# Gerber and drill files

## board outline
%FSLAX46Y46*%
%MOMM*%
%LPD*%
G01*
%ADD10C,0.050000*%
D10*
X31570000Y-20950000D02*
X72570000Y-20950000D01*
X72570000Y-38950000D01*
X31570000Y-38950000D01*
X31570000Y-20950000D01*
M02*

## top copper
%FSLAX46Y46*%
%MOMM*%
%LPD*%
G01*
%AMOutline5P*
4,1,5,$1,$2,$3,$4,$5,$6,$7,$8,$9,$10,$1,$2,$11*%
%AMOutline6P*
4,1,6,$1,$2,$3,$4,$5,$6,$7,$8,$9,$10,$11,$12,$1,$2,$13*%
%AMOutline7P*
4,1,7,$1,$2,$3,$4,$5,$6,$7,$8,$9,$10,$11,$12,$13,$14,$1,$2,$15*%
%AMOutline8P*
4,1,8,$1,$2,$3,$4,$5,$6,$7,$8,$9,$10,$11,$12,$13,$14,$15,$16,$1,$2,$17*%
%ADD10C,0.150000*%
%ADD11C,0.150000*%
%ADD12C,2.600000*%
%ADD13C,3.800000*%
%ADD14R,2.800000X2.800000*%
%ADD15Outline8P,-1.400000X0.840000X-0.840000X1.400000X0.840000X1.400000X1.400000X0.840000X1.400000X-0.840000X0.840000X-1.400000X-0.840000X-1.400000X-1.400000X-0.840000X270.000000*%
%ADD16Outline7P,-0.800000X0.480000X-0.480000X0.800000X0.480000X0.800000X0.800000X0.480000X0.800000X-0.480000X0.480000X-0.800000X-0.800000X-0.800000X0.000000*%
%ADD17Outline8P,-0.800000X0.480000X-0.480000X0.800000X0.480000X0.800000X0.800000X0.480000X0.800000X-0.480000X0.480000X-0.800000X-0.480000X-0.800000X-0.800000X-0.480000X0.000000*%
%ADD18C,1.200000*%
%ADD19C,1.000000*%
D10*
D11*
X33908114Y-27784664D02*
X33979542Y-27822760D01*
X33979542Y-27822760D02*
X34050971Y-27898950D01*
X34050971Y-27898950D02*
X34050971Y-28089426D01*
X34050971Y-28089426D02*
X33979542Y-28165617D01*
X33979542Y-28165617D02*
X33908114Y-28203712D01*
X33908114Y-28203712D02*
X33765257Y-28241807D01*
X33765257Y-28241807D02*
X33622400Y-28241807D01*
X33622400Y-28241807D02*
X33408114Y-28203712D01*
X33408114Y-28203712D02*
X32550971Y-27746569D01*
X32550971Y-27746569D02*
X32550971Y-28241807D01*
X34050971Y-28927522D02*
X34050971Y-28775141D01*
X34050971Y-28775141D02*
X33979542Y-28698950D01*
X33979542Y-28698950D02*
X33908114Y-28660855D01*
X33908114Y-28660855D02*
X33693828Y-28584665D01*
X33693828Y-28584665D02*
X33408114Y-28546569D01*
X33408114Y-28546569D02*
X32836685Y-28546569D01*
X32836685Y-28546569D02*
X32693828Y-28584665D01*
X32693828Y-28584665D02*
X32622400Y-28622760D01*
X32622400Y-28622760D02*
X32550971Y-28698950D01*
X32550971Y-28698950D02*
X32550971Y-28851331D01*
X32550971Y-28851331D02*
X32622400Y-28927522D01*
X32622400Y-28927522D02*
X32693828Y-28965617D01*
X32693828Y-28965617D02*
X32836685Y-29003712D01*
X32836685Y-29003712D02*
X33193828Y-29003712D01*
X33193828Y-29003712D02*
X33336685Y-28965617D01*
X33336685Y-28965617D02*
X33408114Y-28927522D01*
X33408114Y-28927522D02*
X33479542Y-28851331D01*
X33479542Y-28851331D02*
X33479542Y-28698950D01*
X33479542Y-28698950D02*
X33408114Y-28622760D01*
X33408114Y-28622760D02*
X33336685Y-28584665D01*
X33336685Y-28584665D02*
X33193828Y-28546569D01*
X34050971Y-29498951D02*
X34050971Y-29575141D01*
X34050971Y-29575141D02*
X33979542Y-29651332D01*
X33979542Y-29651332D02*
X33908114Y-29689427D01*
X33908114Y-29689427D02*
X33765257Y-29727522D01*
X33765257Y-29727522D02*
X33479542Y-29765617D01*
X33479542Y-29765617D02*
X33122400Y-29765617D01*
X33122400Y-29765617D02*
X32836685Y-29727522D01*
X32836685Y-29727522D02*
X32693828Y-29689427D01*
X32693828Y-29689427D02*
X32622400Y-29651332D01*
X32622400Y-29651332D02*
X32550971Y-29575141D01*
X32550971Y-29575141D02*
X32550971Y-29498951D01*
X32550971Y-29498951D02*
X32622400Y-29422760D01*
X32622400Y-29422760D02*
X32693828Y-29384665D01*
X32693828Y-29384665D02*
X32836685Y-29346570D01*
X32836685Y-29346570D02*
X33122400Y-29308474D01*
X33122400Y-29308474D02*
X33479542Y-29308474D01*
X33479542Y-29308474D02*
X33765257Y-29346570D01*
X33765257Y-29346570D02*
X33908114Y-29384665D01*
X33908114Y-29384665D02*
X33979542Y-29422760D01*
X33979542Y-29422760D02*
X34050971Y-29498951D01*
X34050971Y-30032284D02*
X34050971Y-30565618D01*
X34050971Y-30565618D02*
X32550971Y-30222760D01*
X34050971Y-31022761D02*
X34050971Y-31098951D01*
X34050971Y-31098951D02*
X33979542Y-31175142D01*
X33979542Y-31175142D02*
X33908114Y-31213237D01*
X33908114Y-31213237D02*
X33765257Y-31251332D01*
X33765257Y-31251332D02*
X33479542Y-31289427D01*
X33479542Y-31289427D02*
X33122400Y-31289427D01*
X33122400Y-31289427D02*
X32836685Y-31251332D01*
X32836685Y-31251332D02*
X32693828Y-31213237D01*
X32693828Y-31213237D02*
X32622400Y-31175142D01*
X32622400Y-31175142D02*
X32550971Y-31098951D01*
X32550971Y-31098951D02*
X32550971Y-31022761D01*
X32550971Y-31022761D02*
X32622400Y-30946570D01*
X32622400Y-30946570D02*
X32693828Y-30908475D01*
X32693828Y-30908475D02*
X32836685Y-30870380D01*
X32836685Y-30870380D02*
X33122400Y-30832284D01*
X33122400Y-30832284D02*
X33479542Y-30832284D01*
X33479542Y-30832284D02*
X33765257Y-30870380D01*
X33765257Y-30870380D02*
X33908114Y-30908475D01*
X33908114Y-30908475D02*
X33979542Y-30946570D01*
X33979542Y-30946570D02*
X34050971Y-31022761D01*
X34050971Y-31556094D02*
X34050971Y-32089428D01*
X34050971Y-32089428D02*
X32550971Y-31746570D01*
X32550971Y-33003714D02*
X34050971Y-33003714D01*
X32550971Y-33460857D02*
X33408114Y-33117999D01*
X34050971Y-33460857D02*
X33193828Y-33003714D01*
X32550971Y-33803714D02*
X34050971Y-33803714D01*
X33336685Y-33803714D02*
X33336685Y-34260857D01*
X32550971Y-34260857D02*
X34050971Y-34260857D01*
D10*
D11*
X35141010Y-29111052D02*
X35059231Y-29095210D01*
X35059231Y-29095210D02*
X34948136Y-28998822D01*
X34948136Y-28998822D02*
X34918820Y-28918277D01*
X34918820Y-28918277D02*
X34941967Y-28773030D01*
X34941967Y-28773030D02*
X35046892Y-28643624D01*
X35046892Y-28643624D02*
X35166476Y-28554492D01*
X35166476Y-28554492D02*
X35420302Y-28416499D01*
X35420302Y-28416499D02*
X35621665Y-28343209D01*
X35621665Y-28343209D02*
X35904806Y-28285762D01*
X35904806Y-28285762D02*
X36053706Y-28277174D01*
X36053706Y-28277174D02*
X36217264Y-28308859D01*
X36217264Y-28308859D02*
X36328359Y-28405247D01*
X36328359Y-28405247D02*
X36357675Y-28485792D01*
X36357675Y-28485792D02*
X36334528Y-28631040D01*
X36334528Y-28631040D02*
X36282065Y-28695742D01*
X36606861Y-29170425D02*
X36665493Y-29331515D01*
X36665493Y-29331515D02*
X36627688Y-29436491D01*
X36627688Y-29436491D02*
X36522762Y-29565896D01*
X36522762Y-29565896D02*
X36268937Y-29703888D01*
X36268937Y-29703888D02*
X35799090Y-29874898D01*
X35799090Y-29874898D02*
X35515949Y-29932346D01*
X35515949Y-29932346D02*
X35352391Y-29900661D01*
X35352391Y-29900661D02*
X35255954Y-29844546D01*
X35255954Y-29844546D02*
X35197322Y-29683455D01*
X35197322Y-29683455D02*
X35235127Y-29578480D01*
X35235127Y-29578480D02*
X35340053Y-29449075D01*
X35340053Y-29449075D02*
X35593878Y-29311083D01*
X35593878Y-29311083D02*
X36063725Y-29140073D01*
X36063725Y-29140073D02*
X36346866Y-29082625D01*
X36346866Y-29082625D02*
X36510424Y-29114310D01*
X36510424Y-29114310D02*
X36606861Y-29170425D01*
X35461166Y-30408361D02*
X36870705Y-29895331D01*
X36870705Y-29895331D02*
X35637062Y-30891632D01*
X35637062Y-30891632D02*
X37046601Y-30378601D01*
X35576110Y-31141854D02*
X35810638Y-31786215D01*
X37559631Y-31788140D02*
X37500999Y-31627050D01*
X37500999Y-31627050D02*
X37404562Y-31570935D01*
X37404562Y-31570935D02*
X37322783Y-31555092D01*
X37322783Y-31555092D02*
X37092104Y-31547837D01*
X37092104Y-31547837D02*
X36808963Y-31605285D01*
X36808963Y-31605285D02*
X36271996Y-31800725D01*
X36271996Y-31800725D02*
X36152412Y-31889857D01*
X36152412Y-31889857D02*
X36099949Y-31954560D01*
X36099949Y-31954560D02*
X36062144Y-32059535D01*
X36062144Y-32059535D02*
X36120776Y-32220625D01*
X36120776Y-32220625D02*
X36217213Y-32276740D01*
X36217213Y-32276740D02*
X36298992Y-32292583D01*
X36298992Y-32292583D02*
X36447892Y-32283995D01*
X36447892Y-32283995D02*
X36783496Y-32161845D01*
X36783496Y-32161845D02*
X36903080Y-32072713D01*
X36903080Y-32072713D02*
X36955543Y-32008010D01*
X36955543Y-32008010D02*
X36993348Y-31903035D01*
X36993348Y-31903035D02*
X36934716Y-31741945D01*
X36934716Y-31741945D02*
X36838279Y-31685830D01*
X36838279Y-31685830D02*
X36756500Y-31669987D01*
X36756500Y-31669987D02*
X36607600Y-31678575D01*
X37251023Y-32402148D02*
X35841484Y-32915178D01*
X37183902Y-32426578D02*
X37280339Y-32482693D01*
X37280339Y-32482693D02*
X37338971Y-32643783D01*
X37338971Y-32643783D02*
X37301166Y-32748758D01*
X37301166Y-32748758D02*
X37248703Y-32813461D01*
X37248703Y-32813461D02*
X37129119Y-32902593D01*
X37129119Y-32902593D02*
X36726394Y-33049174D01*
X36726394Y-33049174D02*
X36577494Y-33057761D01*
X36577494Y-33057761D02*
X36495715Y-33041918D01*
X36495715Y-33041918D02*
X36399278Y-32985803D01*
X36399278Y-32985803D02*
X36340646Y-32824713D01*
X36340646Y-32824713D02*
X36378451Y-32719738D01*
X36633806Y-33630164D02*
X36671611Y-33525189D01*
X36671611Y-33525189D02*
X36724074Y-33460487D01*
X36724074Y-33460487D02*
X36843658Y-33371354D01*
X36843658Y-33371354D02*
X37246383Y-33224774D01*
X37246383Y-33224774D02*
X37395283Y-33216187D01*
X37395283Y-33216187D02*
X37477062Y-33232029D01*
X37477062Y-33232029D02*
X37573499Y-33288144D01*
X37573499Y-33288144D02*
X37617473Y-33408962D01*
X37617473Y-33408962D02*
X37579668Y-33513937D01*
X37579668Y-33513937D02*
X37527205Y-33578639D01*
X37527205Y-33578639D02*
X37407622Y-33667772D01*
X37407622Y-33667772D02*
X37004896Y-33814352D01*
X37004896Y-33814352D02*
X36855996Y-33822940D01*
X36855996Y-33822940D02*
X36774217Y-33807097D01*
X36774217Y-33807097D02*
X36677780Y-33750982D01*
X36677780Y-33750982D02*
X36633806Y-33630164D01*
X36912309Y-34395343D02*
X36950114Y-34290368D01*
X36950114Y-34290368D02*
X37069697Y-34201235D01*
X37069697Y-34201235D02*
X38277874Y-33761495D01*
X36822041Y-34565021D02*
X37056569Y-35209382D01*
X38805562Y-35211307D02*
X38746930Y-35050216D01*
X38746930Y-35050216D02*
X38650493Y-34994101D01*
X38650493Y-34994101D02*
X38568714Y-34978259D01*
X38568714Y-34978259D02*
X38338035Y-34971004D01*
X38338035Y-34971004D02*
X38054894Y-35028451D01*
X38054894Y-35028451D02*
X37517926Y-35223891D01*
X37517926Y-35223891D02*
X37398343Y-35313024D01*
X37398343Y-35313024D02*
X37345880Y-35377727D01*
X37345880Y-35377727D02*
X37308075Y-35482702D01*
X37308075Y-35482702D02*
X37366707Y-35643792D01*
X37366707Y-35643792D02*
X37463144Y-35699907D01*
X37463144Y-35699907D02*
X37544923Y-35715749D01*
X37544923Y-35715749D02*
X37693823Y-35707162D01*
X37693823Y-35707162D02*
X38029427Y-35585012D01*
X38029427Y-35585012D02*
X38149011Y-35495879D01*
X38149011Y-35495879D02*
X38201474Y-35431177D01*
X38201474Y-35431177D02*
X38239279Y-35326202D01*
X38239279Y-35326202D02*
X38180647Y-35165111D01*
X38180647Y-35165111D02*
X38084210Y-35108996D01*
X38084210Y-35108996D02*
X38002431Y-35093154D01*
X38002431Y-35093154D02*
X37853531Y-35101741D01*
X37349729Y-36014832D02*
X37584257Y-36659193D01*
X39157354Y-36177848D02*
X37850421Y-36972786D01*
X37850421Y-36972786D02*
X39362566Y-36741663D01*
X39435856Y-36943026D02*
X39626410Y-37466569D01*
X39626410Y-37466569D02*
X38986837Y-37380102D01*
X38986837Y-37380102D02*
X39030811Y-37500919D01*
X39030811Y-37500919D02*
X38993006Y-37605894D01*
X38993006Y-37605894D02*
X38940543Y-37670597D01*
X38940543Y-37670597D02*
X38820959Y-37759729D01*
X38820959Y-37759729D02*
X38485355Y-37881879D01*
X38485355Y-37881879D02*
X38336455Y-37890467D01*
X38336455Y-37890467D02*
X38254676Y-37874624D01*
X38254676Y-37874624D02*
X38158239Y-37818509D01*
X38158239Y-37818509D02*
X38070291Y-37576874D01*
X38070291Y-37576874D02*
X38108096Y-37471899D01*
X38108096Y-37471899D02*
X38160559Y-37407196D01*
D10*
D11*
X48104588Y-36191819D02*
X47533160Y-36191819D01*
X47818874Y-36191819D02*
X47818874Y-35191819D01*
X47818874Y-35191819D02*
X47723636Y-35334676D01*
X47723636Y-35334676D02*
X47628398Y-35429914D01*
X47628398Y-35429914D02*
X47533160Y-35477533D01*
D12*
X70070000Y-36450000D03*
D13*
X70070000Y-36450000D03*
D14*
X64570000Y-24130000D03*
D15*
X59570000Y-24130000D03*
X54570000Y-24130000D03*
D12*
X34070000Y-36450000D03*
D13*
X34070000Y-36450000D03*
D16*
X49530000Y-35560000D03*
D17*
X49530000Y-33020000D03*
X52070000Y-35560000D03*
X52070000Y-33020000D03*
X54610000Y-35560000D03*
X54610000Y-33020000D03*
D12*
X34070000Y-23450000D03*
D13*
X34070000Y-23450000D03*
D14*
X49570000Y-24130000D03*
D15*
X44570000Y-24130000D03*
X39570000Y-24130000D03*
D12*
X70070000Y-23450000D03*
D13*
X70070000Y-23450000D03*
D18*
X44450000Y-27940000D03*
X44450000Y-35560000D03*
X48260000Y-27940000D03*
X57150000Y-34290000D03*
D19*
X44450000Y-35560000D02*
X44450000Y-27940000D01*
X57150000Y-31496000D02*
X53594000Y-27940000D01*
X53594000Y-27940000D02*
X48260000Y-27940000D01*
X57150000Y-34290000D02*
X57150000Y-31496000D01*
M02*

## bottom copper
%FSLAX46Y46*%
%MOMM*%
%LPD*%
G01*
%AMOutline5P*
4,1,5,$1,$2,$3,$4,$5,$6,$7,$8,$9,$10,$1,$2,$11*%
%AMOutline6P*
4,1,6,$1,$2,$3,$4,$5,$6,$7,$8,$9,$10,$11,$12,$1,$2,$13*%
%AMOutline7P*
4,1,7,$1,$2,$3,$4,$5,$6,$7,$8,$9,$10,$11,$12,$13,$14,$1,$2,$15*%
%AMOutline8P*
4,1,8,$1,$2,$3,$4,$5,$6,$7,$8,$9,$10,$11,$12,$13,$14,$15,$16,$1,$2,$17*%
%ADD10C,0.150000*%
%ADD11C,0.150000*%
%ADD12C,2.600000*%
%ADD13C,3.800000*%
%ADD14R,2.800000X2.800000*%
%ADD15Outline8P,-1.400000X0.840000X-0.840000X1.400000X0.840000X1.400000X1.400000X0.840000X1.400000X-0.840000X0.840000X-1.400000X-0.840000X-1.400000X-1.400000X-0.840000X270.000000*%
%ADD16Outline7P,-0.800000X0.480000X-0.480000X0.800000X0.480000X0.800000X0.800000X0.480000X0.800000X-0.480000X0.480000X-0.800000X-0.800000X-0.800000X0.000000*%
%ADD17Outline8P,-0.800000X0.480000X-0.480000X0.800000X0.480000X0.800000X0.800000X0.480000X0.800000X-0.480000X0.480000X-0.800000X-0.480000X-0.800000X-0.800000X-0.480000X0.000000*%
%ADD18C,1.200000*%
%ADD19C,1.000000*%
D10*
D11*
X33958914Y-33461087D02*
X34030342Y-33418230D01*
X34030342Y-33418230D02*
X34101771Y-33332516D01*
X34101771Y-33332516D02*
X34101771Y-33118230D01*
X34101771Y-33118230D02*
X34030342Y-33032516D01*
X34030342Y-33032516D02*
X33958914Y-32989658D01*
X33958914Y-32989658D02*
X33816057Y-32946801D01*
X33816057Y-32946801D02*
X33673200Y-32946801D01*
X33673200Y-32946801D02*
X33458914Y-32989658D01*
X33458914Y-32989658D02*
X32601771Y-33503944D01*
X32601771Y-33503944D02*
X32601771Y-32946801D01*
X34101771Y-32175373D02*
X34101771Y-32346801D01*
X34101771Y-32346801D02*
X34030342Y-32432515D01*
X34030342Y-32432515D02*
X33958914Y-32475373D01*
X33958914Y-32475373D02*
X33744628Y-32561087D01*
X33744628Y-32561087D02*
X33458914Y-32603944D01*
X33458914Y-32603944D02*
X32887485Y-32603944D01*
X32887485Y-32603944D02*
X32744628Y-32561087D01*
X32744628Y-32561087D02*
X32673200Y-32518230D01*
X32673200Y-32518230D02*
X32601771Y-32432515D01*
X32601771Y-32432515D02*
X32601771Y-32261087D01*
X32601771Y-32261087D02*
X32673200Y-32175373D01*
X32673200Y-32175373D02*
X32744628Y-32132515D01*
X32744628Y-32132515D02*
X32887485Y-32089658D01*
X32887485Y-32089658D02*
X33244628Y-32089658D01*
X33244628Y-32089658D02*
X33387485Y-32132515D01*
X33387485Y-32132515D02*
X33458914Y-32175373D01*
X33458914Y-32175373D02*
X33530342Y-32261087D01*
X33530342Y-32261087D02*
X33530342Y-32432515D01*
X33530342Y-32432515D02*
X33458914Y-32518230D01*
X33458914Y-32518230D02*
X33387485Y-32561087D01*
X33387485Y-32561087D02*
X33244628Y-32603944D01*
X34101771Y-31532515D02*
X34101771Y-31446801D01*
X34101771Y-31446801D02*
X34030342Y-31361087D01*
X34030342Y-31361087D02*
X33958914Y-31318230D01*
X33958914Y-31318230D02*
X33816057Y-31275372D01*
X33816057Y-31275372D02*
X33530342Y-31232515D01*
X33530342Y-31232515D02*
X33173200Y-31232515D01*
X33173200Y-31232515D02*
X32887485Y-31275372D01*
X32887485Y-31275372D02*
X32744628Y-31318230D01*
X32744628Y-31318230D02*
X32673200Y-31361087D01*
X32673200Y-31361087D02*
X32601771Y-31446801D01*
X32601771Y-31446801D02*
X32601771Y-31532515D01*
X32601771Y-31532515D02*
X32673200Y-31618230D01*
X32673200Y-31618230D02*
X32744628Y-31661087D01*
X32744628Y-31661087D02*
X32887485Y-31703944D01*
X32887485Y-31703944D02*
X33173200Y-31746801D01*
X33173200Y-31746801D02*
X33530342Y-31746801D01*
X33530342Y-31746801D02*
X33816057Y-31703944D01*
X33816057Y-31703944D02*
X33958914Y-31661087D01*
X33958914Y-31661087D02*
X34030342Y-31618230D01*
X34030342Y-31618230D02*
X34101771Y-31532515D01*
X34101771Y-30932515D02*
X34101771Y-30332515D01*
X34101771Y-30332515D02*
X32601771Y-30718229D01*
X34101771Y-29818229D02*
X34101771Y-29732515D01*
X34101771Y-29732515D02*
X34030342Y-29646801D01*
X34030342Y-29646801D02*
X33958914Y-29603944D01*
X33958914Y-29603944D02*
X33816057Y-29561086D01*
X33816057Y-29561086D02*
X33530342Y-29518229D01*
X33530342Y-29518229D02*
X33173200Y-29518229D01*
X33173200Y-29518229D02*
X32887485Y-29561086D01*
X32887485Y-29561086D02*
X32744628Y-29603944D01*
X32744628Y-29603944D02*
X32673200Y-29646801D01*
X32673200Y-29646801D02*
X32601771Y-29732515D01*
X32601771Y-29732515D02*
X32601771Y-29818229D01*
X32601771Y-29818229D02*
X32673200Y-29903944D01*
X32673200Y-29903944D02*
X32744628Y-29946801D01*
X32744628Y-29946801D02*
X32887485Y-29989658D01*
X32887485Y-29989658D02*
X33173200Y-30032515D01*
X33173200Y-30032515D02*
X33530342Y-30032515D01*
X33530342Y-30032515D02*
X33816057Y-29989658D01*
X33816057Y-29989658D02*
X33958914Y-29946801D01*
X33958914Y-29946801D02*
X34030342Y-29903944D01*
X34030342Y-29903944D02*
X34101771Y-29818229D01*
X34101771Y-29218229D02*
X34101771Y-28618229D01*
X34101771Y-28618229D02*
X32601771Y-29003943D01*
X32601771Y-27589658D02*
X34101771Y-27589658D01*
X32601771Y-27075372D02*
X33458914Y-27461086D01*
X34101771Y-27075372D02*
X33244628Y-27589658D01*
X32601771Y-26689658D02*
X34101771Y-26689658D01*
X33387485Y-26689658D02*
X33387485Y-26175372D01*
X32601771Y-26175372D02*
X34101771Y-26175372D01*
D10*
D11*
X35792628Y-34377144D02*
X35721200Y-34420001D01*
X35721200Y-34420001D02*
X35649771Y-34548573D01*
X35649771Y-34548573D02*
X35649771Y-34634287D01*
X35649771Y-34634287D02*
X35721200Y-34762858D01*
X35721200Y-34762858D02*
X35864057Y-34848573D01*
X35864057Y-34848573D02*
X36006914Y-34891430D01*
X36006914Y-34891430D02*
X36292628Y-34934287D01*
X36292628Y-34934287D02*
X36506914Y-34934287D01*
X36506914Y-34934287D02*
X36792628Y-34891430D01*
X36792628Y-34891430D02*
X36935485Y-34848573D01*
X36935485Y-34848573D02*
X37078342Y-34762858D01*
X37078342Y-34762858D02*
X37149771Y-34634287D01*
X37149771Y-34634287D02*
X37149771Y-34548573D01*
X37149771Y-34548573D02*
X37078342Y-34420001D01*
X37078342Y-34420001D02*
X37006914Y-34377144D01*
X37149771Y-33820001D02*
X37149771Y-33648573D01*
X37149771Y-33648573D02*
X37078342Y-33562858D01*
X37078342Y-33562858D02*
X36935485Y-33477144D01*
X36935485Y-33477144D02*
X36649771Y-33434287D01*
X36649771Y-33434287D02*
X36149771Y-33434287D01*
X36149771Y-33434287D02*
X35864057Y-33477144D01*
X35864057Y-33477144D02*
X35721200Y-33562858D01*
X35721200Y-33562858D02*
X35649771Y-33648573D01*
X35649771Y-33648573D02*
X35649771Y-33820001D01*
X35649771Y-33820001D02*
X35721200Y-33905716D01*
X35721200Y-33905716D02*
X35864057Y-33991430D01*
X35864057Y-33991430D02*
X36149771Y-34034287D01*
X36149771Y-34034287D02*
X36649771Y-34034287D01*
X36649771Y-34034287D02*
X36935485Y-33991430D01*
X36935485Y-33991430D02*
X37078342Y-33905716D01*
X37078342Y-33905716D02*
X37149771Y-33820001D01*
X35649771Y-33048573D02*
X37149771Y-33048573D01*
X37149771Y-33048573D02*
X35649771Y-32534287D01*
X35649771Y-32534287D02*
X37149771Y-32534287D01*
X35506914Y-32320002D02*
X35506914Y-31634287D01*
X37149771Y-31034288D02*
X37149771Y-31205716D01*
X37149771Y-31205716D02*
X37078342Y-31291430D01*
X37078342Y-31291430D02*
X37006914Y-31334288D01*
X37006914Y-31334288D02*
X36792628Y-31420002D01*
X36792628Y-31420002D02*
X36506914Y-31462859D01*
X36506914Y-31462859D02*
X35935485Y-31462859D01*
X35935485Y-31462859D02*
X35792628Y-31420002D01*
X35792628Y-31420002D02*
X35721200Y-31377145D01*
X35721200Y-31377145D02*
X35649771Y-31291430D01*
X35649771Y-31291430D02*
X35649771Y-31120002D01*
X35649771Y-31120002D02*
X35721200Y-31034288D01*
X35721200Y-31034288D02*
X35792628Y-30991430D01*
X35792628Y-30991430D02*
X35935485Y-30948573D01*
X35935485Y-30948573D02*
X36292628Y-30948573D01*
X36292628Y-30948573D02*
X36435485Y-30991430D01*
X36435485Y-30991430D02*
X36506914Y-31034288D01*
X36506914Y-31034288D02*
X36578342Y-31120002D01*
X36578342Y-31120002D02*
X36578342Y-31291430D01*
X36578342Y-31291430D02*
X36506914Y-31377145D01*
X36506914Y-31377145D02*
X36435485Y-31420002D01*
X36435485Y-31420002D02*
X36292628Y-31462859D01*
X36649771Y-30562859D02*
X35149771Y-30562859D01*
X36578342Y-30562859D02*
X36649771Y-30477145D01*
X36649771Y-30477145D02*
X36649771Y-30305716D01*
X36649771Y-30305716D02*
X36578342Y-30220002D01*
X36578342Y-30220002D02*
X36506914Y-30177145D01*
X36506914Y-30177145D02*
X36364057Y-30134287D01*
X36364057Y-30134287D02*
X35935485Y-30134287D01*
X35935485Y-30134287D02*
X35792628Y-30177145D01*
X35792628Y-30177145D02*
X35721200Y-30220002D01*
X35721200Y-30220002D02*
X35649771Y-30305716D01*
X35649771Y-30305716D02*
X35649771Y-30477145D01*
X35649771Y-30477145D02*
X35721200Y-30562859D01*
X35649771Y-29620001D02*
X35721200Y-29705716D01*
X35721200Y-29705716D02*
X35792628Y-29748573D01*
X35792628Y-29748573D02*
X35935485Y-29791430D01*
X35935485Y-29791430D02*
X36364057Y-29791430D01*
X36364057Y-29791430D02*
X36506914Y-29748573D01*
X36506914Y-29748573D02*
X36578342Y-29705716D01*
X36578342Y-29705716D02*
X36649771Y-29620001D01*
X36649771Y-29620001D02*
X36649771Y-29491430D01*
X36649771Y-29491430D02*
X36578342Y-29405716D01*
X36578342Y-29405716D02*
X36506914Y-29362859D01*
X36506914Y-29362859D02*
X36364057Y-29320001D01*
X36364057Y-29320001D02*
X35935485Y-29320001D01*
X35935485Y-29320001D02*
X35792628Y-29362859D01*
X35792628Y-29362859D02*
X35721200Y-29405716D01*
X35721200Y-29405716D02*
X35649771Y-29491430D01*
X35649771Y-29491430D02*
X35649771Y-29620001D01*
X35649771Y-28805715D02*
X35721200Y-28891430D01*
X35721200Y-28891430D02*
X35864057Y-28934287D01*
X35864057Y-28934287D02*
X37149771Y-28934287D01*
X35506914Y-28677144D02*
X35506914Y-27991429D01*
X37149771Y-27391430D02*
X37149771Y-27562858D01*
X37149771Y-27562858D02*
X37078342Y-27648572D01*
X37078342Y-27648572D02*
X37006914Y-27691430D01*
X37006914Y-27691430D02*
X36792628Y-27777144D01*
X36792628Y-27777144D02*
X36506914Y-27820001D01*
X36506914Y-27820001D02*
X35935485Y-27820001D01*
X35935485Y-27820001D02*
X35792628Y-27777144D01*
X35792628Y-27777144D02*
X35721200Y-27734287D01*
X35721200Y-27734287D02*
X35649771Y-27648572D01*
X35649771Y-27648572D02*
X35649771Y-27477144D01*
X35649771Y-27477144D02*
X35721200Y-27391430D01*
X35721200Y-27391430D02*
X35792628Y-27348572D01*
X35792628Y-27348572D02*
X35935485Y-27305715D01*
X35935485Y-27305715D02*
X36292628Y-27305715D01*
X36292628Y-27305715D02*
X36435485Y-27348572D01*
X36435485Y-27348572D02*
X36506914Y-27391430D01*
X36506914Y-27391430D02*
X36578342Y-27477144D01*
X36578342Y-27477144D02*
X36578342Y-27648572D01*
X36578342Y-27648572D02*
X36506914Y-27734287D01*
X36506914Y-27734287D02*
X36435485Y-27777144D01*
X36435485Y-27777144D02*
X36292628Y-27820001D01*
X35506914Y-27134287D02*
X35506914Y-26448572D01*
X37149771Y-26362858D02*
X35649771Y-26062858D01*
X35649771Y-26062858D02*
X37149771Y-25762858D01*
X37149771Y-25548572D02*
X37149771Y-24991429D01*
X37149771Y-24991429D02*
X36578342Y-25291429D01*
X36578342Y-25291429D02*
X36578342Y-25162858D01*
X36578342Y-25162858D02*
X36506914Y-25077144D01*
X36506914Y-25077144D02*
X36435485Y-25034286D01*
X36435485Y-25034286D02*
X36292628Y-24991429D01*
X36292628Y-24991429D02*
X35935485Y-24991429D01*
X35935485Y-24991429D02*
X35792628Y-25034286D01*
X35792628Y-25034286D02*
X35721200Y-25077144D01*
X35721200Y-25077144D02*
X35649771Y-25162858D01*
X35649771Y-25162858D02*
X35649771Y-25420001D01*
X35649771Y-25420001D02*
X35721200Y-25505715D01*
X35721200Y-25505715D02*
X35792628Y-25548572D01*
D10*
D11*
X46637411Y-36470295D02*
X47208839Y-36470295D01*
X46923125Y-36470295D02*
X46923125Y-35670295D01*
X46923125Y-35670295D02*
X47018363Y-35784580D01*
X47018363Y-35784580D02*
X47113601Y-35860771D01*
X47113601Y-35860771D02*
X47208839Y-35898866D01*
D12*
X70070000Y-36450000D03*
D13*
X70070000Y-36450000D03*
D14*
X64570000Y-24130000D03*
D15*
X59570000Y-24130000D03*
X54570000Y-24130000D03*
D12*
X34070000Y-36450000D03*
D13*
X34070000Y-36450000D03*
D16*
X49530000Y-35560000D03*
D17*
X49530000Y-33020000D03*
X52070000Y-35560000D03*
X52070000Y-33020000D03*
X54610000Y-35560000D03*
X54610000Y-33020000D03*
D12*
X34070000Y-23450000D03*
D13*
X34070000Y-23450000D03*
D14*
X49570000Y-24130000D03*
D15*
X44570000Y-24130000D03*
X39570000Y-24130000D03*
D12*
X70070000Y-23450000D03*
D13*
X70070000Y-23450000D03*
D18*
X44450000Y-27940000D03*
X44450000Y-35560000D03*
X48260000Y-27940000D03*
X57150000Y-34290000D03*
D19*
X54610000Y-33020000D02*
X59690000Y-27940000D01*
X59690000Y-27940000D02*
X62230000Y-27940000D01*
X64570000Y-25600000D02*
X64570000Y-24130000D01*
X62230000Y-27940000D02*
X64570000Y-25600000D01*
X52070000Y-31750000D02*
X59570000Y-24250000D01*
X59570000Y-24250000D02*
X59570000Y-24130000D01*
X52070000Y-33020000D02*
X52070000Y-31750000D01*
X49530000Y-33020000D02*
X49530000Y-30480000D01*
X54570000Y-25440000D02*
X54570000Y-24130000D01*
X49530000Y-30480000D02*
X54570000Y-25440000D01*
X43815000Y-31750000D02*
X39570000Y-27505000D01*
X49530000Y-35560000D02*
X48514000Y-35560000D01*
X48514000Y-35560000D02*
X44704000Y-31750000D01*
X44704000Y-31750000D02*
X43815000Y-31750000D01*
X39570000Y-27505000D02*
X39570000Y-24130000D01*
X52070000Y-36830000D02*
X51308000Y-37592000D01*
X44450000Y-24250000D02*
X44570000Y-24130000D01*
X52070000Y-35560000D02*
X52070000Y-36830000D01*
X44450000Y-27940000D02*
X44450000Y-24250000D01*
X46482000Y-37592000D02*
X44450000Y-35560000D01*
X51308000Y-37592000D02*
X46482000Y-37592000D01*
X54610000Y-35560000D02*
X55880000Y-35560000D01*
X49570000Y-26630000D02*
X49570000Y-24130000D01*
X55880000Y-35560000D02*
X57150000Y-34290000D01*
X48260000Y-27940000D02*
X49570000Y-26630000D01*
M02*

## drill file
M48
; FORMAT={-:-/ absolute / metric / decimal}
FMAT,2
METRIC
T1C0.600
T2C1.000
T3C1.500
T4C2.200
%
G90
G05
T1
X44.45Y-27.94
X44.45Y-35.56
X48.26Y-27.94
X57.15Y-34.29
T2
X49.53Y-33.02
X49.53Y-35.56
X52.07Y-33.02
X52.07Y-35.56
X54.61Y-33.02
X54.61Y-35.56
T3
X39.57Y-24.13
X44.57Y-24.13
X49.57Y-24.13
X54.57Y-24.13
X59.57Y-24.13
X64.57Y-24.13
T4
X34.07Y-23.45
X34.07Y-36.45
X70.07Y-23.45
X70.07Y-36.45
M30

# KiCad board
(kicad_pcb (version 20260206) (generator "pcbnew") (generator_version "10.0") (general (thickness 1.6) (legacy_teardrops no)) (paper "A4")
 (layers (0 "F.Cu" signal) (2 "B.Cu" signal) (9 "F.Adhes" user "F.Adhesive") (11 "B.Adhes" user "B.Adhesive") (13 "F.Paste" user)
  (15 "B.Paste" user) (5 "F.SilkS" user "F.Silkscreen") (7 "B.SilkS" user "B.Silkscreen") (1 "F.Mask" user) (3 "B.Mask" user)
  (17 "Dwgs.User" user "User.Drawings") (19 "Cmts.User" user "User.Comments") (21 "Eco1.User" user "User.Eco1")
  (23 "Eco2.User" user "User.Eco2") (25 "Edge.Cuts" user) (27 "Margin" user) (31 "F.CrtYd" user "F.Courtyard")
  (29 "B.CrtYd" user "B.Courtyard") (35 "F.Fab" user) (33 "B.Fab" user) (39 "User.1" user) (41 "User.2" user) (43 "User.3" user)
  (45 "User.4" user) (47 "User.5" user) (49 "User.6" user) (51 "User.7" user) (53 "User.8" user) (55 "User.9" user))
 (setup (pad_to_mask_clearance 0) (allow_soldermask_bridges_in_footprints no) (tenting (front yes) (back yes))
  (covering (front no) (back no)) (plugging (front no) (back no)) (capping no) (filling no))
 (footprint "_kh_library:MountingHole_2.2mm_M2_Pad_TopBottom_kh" (layer "F.Cu") (at 70.07 36.45)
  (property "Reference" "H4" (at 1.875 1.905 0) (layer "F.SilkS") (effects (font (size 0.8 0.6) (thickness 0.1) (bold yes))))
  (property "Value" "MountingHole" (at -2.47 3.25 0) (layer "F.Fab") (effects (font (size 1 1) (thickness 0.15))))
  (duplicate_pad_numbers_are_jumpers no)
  (pad "1" thru_hole circle (at 0 0) (size 2.6 2.6) (drill 2.2) (layers "*.Cu" "*.Mask") (remove_unused_layers no))
  (pad "1" connect circle (at 0 0) (size 3.8 3.8) (layers "F.Cu" "F.Mask"))
  (pad "1" connect circle (at 0 0) (size 3.8 3.8) (layers "B.Cu" "B.Mask")))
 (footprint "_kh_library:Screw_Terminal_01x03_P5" (layer "F.Cu") (at 64.57 24.13 -90)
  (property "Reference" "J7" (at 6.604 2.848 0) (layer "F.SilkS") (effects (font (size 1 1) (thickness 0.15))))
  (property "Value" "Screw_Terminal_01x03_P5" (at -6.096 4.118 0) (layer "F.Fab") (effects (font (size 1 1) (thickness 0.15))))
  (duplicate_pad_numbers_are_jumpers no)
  (pad "1" thru_hole rect (at 0 0 270) (size 2.8 2.8) (drill 1.5) (layers "*.Cu" "*.Mask") (remove_unused_layers no) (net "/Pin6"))
  (pad "2" thru_hole roundrect (at 0 5 270) (size 2.8 2.8) (drill 1.5) (layers "*.Cu" "*.Mask") (remove_unused_layers no)
   (roundrect_rratio 0) (chamfer_ratio 0.2) (chamfer top_left top_right bottom_left bottom_right) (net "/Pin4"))
  (pad "3" thru_hole roundrect (at 0 10 270) (size 2.8 2.8) (drill 1.5) (layers "*.Cu" "*.Mask") (remove_unused_layers no)
   (roundrect_rratio 0) (chamfer_ratio 0.2) (chamfer top_left top_right bottom_left bottom_right) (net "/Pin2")))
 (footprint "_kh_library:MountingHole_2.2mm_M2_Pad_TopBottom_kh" (layer "F.Cu") (at 34.07 36.45)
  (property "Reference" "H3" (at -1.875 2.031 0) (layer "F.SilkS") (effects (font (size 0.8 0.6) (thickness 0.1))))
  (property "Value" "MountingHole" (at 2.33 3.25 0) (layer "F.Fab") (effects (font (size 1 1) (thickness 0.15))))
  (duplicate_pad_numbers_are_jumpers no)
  (pad "1" thru_hole circle (at 0 0) (size 2.6 2.6) (drill 2.2) (layers "*.Cu" "*.Mask") (remove_unused_layers no))
  (pad "1" connect circle (at 0 0) (size 3.8 3.8) (layers "F.Cu" "F.Mask"))
  (pad "1" connect circle (at 0 0) (size 3.8 3.8) (layers "B.Cu" "B.Mask")))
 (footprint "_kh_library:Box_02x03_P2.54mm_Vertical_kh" (layer "F.Cu") (at 49.53 35.56)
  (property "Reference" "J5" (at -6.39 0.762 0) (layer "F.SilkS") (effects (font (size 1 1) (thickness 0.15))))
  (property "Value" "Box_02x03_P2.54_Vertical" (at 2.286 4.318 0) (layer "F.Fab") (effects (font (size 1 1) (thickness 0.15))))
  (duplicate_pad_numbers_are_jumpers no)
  (pad "1" thru_hole roundrect (at 0 0) (size 1.6 1.6) (drill 1) (layers "*.Cu" "*.Mask") (remove_unused_layers no) (roundrect_rratio 0)
   (chamfer_ratio 0.2) (chamfer top_left top_right bottom_right) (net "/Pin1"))
  (pad "2" thru_hole roundrect (at 0 -2.54) (size 1.6 1.6) (drill 1) (layers "*.Cu" "*.Mask") (remove_unused_layers no) (roundrect_rratio 0)
   (chamfer_ratio 0.2) (chamfer top_left top_right bottom_left bottom_right) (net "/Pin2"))
  (pad "3" thru_hole roundrect (at 2.54 0) (size 1.6 1.6) (drill 1) (layers "*.Cu" "*.Mask") (remove_unused_layers no) (roundrect_rratio 0)
   (chamfer_ratio 0.2) (chamfer top_left top_right bottom_left bottom_right) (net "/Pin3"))
  (pad "4" thru_hole roundrect (at 2.54 -2.54) (size 1.6 1.6) (drill 1) (layers "*.Cu" "*.Mask") (remove_unused_layers no)
   (roundrect_rratio 0) (chamfer_ratio 0.2) (chamfer top_left top_right bottom_left bottom_right) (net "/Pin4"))
  (pad "5" thru_hole roundrect (at 5.08 0) (size 1.6 1.6) (drill 1) (layers "*.Cu" "*.Mask") (remove_unused_layers no) (roundrect_rratio 0)
   (chamfer_ratio 0.2) (chamfer top_left top_right bottom_left bottom_right) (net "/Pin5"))
  (pad "6" thru_hole roundrect (at 5.08 -2.54) (size 1.6 1.6) (drill 1) (layers "*.Cu" "*.Mask") (remove_unused_layers no)
   (roundrect_rratio 0) (chamfer_ratio 0.2) (chamfer top_left top_right bottom_left bottom_right) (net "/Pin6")))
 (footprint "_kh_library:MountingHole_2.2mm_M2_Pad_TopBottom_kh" (layer "F.Cu") (at 34.07 23.45)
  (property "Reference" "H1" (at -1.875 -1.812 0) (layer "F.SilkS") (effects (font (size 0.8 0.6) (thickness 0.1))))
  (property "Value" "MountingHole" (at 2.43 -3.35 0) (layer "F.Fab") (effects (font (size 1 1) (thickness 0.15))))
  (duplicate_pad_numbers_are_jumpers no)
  (pad "1" thru_hole circle (at 0 0) (size 2.6 2.6) (drill 2.2) (layers "*.Cu" "*.Mask") (remove_unused_layers no))
  (pad "1" connect circle (at 0 0) (size 3.8 3.8) (layers "F.Cu" "F.Mask"))
  (pad "1" connect circle (at 0 0) (size 3.8 3.8) (layers "B.Cu" "B.Mask")))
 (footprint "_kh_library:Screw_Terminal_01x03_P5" (layer "F.Cu") (at 49.57 24.13 -90)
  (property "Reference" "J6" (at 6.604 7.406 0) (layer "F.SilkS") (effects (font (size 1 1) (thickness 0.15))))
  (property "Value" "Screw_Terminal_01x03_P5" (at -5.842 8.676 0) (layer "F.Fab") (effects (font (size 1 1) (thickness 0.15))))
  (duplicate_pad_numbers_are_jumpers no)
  (pad "1" thru_hole rect (at 0 0 270) (size 2.8 2.8) (drill 1.5) (layers "*.Cu" "*.Mask") (remove_unused_layers no) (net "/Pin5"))
  (pad "2" thru_hole roundrect (at 0 5 270) (size 2.8 2.8) (drill 1.5) (layers "*.Cu" "*.Mask") (remove_unused_layers no)
   (roundrect_rratio 0) (chamfer_ratio 0.2) (chamfer top_left top_right bottom_left bottom_right) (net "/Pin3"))
  (pad "3" thru_hole roundrect (at 0 10 270) (size 2.8 2.8) (drill 1.5) (layers "*.Cu" "*.Mask") (remove_unused_layers no)
   (roundrect_rratio 0) (chamfer_ratio 0.2) (chamfer top_left top_right bottom_left bottom_right) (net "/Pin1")))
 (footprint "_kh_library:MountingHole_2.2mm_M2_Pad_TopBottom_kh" (layer "F.Cu") (at 70.07 23.45)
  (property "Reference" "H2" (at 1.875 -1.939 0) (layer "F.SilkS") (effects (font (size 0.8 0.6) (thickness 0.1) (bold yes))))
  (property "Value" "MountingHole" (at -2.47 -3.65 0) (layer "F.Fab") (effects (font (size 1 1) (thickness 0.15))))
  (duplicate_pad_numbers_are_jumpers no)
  (pad "1" thru_hole circle (at 0 0) (size 2.6 2.6) (drill 2.2) (layers "*.Cu" "*.Mask") (remove_unused_layers no))
  (pad "1" connect circle (at 0 0) (size 3.8 3.8) (layers "F.Cu" "F.Mask"))
  (pad "1" connect circle (at 0 0) (size 3.8 3.8) (layers "B.Cu" "B.Mask")))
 (gr_rect (start 31.57 20.95) (end 72.57 38.95) (stroke (width 0.05) (type default)) (fill no) (layer "Edge.Cuts"))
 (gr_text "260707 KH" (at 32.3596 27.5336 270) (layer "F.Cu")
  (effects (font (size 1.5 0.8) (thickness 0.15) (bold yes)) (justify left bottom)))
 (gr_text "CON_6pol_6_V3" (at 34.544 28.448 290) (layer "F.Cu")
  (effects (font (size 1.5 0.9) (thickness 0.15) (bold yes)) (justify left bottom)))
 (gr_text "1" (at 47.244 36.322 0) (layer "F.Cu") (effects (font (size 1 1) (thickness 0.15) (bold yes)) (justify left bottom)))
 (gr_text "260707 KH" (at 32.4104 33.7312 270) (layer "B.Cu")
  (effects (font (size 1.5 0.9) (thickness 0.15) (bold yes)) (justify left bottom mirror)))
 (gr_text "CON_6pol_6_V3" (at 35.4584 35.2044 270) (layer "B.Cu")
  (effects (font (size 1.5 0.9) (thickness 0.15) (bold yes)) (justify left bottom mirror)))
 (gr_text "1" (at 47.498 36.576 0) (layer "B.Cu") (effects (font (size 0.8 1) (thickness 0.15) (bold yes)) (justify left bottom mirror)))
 (segment (start 54.61 33.02) (end 59.69 27.94) (width 1) (layer "B.Cu") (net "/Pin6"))
 (segment (start 59.69 27.94) (end 62.23 27.94) (width 1) (layer "B.Cu") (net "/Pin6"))
 (segment (start 64.57 25.6) (end 64.57 24.13) (width 1) (layer "B.Cu") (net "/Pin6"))
 (segment (start 62.23 27.94) (end 64.57 25.6) (width 1) (layer "B.Cu") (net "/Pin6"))
 (segment (start 52.07 31.75) (end 59.57 24.25) (width 1) (layer "B.Cu") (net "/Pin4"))
 (segment (start 59.57 24.25) (end 59.57 24.13) (width 1) (layer "B.Cu") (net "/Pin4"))
 (segment (start 52.07 33.02) (end 52.07 31.75) (width 1) (layer "B.Cu") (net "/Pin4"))
 (segment (start 49.53 33.02) (end 49.53 30.48) (width 1) (layer "B.Cu") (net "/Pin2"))
 (segment (start 54.57 25.44) (end 54.57 24.13) (width 1) (layer "B.Cu") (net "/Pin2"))
 (segment (start 49.53 30.48) (end 54.57 25.44) (width 1) (layer "B.Cu") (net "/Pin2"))
 (segment (start 43.815 31.75) (end 39.57 27.505) (width 1) (layer "B.Cu") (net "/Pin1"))
 (segment (start 49.53 35.56) (end 48.514 35.56) (width 1) (layer "B.Cu") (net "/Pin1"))
 (segment (start 48.514 35.56) (end 44.704 31.75) (width 1) (layer "B.Cu") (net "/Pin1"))
 (segment (start 44.704 31.75) (end 43.815 31.75) (width 1) (layer "B.Cu") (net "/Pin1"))
 (segment (start 39.57 27.505) (end 39.57 24.13) (width 1) (layer "B.Cu") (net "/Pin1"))
 (segment (start 44.45 35.56) (end 44.45 27.94) (width 1) (layer "F.Cu") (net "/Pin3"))
 (via (at 44.45 27.94) (size 1.2) (drill 0.6) (layers "F.Cu" "B.Cu") (capping no) (covering (front no) (back no))
  (plugging (front no) (back no)) (filling no) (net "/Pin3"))
 (via (at 44.45 35.56) (size 1.2) (drill 0.6) (layers "F.Cu" "B.Cu") (capping no) (covering (front no) (back no))
  (plugging (front no) (back no)) (filling no) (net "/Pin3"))
 (segment (start 52.07 36.83) (end 51.308 37.592) (width 1) (layer "B.Cu") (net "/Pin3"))
 (segment (start 44.45 24.25) (end 44.57 24.13) (width 1) (layer "B.Cu") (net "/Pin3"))
 (segment (start 52.07 35.56) (end 52.07 36.83) (width 1) (layer "B.Cu") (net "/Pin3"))
 (segment (start 44.45 27.94) (end 44.45 24.25) (width 1) (layer "B.Cu") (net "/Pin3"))
 (segment (start 46.482 37.592) (end 44.45 35.56) (width 1) (layer "B.Cu") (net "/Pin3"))
 (segment (start 51.308 37.592) (end 46.482 37.592) (width 1) (layer "B.Cu") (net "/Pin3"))
 (segment (start 57.15 31.496) (end 53.594 27.94) (width 1) (layer "F.Cu") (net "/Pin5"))
 (segment (start 53.594 27.94) (end 48.26 27.94) (width 1) (layer "F.Cu") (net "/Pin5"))
 (segment (start 57.15 34.29) (end 57.15 31.496) (width 1) (layer "F.Cu") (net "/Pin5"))
 (via (at 48.26 27.94) (size 1.2) (drill 0.6) (layers "F.Cu" "B.Cu") (capping no) (covering (front no) (back no))
  (plugging (front no) (back no)) (filling no) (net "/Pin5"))
 (via (at 57.15 34.29) (size 1.2) (drill 0.6) (layers "F.Cu" "B.Cu") (capping no) (covering (front no) (back no))
  (plugging (front no) (back no)) (filling no) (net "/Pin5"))
 (segment (start 54.61 35.56) (end 55.88 35.56) (width 1) (layer "B.Cu") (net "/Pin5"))
 (segment (start 49.57 26.63) (end 49.57 24.13) (width 1) (layer "B.Cu") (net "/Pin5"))
 (segment (start 55.88 35.56) (end 57.15 34.29) (width 1) (layer "B.Cu") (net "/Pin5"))
 (segment (start 48.26 27.94) (end 49.57 26.63) (width 1) (layer "B.Cu") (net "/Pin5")))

